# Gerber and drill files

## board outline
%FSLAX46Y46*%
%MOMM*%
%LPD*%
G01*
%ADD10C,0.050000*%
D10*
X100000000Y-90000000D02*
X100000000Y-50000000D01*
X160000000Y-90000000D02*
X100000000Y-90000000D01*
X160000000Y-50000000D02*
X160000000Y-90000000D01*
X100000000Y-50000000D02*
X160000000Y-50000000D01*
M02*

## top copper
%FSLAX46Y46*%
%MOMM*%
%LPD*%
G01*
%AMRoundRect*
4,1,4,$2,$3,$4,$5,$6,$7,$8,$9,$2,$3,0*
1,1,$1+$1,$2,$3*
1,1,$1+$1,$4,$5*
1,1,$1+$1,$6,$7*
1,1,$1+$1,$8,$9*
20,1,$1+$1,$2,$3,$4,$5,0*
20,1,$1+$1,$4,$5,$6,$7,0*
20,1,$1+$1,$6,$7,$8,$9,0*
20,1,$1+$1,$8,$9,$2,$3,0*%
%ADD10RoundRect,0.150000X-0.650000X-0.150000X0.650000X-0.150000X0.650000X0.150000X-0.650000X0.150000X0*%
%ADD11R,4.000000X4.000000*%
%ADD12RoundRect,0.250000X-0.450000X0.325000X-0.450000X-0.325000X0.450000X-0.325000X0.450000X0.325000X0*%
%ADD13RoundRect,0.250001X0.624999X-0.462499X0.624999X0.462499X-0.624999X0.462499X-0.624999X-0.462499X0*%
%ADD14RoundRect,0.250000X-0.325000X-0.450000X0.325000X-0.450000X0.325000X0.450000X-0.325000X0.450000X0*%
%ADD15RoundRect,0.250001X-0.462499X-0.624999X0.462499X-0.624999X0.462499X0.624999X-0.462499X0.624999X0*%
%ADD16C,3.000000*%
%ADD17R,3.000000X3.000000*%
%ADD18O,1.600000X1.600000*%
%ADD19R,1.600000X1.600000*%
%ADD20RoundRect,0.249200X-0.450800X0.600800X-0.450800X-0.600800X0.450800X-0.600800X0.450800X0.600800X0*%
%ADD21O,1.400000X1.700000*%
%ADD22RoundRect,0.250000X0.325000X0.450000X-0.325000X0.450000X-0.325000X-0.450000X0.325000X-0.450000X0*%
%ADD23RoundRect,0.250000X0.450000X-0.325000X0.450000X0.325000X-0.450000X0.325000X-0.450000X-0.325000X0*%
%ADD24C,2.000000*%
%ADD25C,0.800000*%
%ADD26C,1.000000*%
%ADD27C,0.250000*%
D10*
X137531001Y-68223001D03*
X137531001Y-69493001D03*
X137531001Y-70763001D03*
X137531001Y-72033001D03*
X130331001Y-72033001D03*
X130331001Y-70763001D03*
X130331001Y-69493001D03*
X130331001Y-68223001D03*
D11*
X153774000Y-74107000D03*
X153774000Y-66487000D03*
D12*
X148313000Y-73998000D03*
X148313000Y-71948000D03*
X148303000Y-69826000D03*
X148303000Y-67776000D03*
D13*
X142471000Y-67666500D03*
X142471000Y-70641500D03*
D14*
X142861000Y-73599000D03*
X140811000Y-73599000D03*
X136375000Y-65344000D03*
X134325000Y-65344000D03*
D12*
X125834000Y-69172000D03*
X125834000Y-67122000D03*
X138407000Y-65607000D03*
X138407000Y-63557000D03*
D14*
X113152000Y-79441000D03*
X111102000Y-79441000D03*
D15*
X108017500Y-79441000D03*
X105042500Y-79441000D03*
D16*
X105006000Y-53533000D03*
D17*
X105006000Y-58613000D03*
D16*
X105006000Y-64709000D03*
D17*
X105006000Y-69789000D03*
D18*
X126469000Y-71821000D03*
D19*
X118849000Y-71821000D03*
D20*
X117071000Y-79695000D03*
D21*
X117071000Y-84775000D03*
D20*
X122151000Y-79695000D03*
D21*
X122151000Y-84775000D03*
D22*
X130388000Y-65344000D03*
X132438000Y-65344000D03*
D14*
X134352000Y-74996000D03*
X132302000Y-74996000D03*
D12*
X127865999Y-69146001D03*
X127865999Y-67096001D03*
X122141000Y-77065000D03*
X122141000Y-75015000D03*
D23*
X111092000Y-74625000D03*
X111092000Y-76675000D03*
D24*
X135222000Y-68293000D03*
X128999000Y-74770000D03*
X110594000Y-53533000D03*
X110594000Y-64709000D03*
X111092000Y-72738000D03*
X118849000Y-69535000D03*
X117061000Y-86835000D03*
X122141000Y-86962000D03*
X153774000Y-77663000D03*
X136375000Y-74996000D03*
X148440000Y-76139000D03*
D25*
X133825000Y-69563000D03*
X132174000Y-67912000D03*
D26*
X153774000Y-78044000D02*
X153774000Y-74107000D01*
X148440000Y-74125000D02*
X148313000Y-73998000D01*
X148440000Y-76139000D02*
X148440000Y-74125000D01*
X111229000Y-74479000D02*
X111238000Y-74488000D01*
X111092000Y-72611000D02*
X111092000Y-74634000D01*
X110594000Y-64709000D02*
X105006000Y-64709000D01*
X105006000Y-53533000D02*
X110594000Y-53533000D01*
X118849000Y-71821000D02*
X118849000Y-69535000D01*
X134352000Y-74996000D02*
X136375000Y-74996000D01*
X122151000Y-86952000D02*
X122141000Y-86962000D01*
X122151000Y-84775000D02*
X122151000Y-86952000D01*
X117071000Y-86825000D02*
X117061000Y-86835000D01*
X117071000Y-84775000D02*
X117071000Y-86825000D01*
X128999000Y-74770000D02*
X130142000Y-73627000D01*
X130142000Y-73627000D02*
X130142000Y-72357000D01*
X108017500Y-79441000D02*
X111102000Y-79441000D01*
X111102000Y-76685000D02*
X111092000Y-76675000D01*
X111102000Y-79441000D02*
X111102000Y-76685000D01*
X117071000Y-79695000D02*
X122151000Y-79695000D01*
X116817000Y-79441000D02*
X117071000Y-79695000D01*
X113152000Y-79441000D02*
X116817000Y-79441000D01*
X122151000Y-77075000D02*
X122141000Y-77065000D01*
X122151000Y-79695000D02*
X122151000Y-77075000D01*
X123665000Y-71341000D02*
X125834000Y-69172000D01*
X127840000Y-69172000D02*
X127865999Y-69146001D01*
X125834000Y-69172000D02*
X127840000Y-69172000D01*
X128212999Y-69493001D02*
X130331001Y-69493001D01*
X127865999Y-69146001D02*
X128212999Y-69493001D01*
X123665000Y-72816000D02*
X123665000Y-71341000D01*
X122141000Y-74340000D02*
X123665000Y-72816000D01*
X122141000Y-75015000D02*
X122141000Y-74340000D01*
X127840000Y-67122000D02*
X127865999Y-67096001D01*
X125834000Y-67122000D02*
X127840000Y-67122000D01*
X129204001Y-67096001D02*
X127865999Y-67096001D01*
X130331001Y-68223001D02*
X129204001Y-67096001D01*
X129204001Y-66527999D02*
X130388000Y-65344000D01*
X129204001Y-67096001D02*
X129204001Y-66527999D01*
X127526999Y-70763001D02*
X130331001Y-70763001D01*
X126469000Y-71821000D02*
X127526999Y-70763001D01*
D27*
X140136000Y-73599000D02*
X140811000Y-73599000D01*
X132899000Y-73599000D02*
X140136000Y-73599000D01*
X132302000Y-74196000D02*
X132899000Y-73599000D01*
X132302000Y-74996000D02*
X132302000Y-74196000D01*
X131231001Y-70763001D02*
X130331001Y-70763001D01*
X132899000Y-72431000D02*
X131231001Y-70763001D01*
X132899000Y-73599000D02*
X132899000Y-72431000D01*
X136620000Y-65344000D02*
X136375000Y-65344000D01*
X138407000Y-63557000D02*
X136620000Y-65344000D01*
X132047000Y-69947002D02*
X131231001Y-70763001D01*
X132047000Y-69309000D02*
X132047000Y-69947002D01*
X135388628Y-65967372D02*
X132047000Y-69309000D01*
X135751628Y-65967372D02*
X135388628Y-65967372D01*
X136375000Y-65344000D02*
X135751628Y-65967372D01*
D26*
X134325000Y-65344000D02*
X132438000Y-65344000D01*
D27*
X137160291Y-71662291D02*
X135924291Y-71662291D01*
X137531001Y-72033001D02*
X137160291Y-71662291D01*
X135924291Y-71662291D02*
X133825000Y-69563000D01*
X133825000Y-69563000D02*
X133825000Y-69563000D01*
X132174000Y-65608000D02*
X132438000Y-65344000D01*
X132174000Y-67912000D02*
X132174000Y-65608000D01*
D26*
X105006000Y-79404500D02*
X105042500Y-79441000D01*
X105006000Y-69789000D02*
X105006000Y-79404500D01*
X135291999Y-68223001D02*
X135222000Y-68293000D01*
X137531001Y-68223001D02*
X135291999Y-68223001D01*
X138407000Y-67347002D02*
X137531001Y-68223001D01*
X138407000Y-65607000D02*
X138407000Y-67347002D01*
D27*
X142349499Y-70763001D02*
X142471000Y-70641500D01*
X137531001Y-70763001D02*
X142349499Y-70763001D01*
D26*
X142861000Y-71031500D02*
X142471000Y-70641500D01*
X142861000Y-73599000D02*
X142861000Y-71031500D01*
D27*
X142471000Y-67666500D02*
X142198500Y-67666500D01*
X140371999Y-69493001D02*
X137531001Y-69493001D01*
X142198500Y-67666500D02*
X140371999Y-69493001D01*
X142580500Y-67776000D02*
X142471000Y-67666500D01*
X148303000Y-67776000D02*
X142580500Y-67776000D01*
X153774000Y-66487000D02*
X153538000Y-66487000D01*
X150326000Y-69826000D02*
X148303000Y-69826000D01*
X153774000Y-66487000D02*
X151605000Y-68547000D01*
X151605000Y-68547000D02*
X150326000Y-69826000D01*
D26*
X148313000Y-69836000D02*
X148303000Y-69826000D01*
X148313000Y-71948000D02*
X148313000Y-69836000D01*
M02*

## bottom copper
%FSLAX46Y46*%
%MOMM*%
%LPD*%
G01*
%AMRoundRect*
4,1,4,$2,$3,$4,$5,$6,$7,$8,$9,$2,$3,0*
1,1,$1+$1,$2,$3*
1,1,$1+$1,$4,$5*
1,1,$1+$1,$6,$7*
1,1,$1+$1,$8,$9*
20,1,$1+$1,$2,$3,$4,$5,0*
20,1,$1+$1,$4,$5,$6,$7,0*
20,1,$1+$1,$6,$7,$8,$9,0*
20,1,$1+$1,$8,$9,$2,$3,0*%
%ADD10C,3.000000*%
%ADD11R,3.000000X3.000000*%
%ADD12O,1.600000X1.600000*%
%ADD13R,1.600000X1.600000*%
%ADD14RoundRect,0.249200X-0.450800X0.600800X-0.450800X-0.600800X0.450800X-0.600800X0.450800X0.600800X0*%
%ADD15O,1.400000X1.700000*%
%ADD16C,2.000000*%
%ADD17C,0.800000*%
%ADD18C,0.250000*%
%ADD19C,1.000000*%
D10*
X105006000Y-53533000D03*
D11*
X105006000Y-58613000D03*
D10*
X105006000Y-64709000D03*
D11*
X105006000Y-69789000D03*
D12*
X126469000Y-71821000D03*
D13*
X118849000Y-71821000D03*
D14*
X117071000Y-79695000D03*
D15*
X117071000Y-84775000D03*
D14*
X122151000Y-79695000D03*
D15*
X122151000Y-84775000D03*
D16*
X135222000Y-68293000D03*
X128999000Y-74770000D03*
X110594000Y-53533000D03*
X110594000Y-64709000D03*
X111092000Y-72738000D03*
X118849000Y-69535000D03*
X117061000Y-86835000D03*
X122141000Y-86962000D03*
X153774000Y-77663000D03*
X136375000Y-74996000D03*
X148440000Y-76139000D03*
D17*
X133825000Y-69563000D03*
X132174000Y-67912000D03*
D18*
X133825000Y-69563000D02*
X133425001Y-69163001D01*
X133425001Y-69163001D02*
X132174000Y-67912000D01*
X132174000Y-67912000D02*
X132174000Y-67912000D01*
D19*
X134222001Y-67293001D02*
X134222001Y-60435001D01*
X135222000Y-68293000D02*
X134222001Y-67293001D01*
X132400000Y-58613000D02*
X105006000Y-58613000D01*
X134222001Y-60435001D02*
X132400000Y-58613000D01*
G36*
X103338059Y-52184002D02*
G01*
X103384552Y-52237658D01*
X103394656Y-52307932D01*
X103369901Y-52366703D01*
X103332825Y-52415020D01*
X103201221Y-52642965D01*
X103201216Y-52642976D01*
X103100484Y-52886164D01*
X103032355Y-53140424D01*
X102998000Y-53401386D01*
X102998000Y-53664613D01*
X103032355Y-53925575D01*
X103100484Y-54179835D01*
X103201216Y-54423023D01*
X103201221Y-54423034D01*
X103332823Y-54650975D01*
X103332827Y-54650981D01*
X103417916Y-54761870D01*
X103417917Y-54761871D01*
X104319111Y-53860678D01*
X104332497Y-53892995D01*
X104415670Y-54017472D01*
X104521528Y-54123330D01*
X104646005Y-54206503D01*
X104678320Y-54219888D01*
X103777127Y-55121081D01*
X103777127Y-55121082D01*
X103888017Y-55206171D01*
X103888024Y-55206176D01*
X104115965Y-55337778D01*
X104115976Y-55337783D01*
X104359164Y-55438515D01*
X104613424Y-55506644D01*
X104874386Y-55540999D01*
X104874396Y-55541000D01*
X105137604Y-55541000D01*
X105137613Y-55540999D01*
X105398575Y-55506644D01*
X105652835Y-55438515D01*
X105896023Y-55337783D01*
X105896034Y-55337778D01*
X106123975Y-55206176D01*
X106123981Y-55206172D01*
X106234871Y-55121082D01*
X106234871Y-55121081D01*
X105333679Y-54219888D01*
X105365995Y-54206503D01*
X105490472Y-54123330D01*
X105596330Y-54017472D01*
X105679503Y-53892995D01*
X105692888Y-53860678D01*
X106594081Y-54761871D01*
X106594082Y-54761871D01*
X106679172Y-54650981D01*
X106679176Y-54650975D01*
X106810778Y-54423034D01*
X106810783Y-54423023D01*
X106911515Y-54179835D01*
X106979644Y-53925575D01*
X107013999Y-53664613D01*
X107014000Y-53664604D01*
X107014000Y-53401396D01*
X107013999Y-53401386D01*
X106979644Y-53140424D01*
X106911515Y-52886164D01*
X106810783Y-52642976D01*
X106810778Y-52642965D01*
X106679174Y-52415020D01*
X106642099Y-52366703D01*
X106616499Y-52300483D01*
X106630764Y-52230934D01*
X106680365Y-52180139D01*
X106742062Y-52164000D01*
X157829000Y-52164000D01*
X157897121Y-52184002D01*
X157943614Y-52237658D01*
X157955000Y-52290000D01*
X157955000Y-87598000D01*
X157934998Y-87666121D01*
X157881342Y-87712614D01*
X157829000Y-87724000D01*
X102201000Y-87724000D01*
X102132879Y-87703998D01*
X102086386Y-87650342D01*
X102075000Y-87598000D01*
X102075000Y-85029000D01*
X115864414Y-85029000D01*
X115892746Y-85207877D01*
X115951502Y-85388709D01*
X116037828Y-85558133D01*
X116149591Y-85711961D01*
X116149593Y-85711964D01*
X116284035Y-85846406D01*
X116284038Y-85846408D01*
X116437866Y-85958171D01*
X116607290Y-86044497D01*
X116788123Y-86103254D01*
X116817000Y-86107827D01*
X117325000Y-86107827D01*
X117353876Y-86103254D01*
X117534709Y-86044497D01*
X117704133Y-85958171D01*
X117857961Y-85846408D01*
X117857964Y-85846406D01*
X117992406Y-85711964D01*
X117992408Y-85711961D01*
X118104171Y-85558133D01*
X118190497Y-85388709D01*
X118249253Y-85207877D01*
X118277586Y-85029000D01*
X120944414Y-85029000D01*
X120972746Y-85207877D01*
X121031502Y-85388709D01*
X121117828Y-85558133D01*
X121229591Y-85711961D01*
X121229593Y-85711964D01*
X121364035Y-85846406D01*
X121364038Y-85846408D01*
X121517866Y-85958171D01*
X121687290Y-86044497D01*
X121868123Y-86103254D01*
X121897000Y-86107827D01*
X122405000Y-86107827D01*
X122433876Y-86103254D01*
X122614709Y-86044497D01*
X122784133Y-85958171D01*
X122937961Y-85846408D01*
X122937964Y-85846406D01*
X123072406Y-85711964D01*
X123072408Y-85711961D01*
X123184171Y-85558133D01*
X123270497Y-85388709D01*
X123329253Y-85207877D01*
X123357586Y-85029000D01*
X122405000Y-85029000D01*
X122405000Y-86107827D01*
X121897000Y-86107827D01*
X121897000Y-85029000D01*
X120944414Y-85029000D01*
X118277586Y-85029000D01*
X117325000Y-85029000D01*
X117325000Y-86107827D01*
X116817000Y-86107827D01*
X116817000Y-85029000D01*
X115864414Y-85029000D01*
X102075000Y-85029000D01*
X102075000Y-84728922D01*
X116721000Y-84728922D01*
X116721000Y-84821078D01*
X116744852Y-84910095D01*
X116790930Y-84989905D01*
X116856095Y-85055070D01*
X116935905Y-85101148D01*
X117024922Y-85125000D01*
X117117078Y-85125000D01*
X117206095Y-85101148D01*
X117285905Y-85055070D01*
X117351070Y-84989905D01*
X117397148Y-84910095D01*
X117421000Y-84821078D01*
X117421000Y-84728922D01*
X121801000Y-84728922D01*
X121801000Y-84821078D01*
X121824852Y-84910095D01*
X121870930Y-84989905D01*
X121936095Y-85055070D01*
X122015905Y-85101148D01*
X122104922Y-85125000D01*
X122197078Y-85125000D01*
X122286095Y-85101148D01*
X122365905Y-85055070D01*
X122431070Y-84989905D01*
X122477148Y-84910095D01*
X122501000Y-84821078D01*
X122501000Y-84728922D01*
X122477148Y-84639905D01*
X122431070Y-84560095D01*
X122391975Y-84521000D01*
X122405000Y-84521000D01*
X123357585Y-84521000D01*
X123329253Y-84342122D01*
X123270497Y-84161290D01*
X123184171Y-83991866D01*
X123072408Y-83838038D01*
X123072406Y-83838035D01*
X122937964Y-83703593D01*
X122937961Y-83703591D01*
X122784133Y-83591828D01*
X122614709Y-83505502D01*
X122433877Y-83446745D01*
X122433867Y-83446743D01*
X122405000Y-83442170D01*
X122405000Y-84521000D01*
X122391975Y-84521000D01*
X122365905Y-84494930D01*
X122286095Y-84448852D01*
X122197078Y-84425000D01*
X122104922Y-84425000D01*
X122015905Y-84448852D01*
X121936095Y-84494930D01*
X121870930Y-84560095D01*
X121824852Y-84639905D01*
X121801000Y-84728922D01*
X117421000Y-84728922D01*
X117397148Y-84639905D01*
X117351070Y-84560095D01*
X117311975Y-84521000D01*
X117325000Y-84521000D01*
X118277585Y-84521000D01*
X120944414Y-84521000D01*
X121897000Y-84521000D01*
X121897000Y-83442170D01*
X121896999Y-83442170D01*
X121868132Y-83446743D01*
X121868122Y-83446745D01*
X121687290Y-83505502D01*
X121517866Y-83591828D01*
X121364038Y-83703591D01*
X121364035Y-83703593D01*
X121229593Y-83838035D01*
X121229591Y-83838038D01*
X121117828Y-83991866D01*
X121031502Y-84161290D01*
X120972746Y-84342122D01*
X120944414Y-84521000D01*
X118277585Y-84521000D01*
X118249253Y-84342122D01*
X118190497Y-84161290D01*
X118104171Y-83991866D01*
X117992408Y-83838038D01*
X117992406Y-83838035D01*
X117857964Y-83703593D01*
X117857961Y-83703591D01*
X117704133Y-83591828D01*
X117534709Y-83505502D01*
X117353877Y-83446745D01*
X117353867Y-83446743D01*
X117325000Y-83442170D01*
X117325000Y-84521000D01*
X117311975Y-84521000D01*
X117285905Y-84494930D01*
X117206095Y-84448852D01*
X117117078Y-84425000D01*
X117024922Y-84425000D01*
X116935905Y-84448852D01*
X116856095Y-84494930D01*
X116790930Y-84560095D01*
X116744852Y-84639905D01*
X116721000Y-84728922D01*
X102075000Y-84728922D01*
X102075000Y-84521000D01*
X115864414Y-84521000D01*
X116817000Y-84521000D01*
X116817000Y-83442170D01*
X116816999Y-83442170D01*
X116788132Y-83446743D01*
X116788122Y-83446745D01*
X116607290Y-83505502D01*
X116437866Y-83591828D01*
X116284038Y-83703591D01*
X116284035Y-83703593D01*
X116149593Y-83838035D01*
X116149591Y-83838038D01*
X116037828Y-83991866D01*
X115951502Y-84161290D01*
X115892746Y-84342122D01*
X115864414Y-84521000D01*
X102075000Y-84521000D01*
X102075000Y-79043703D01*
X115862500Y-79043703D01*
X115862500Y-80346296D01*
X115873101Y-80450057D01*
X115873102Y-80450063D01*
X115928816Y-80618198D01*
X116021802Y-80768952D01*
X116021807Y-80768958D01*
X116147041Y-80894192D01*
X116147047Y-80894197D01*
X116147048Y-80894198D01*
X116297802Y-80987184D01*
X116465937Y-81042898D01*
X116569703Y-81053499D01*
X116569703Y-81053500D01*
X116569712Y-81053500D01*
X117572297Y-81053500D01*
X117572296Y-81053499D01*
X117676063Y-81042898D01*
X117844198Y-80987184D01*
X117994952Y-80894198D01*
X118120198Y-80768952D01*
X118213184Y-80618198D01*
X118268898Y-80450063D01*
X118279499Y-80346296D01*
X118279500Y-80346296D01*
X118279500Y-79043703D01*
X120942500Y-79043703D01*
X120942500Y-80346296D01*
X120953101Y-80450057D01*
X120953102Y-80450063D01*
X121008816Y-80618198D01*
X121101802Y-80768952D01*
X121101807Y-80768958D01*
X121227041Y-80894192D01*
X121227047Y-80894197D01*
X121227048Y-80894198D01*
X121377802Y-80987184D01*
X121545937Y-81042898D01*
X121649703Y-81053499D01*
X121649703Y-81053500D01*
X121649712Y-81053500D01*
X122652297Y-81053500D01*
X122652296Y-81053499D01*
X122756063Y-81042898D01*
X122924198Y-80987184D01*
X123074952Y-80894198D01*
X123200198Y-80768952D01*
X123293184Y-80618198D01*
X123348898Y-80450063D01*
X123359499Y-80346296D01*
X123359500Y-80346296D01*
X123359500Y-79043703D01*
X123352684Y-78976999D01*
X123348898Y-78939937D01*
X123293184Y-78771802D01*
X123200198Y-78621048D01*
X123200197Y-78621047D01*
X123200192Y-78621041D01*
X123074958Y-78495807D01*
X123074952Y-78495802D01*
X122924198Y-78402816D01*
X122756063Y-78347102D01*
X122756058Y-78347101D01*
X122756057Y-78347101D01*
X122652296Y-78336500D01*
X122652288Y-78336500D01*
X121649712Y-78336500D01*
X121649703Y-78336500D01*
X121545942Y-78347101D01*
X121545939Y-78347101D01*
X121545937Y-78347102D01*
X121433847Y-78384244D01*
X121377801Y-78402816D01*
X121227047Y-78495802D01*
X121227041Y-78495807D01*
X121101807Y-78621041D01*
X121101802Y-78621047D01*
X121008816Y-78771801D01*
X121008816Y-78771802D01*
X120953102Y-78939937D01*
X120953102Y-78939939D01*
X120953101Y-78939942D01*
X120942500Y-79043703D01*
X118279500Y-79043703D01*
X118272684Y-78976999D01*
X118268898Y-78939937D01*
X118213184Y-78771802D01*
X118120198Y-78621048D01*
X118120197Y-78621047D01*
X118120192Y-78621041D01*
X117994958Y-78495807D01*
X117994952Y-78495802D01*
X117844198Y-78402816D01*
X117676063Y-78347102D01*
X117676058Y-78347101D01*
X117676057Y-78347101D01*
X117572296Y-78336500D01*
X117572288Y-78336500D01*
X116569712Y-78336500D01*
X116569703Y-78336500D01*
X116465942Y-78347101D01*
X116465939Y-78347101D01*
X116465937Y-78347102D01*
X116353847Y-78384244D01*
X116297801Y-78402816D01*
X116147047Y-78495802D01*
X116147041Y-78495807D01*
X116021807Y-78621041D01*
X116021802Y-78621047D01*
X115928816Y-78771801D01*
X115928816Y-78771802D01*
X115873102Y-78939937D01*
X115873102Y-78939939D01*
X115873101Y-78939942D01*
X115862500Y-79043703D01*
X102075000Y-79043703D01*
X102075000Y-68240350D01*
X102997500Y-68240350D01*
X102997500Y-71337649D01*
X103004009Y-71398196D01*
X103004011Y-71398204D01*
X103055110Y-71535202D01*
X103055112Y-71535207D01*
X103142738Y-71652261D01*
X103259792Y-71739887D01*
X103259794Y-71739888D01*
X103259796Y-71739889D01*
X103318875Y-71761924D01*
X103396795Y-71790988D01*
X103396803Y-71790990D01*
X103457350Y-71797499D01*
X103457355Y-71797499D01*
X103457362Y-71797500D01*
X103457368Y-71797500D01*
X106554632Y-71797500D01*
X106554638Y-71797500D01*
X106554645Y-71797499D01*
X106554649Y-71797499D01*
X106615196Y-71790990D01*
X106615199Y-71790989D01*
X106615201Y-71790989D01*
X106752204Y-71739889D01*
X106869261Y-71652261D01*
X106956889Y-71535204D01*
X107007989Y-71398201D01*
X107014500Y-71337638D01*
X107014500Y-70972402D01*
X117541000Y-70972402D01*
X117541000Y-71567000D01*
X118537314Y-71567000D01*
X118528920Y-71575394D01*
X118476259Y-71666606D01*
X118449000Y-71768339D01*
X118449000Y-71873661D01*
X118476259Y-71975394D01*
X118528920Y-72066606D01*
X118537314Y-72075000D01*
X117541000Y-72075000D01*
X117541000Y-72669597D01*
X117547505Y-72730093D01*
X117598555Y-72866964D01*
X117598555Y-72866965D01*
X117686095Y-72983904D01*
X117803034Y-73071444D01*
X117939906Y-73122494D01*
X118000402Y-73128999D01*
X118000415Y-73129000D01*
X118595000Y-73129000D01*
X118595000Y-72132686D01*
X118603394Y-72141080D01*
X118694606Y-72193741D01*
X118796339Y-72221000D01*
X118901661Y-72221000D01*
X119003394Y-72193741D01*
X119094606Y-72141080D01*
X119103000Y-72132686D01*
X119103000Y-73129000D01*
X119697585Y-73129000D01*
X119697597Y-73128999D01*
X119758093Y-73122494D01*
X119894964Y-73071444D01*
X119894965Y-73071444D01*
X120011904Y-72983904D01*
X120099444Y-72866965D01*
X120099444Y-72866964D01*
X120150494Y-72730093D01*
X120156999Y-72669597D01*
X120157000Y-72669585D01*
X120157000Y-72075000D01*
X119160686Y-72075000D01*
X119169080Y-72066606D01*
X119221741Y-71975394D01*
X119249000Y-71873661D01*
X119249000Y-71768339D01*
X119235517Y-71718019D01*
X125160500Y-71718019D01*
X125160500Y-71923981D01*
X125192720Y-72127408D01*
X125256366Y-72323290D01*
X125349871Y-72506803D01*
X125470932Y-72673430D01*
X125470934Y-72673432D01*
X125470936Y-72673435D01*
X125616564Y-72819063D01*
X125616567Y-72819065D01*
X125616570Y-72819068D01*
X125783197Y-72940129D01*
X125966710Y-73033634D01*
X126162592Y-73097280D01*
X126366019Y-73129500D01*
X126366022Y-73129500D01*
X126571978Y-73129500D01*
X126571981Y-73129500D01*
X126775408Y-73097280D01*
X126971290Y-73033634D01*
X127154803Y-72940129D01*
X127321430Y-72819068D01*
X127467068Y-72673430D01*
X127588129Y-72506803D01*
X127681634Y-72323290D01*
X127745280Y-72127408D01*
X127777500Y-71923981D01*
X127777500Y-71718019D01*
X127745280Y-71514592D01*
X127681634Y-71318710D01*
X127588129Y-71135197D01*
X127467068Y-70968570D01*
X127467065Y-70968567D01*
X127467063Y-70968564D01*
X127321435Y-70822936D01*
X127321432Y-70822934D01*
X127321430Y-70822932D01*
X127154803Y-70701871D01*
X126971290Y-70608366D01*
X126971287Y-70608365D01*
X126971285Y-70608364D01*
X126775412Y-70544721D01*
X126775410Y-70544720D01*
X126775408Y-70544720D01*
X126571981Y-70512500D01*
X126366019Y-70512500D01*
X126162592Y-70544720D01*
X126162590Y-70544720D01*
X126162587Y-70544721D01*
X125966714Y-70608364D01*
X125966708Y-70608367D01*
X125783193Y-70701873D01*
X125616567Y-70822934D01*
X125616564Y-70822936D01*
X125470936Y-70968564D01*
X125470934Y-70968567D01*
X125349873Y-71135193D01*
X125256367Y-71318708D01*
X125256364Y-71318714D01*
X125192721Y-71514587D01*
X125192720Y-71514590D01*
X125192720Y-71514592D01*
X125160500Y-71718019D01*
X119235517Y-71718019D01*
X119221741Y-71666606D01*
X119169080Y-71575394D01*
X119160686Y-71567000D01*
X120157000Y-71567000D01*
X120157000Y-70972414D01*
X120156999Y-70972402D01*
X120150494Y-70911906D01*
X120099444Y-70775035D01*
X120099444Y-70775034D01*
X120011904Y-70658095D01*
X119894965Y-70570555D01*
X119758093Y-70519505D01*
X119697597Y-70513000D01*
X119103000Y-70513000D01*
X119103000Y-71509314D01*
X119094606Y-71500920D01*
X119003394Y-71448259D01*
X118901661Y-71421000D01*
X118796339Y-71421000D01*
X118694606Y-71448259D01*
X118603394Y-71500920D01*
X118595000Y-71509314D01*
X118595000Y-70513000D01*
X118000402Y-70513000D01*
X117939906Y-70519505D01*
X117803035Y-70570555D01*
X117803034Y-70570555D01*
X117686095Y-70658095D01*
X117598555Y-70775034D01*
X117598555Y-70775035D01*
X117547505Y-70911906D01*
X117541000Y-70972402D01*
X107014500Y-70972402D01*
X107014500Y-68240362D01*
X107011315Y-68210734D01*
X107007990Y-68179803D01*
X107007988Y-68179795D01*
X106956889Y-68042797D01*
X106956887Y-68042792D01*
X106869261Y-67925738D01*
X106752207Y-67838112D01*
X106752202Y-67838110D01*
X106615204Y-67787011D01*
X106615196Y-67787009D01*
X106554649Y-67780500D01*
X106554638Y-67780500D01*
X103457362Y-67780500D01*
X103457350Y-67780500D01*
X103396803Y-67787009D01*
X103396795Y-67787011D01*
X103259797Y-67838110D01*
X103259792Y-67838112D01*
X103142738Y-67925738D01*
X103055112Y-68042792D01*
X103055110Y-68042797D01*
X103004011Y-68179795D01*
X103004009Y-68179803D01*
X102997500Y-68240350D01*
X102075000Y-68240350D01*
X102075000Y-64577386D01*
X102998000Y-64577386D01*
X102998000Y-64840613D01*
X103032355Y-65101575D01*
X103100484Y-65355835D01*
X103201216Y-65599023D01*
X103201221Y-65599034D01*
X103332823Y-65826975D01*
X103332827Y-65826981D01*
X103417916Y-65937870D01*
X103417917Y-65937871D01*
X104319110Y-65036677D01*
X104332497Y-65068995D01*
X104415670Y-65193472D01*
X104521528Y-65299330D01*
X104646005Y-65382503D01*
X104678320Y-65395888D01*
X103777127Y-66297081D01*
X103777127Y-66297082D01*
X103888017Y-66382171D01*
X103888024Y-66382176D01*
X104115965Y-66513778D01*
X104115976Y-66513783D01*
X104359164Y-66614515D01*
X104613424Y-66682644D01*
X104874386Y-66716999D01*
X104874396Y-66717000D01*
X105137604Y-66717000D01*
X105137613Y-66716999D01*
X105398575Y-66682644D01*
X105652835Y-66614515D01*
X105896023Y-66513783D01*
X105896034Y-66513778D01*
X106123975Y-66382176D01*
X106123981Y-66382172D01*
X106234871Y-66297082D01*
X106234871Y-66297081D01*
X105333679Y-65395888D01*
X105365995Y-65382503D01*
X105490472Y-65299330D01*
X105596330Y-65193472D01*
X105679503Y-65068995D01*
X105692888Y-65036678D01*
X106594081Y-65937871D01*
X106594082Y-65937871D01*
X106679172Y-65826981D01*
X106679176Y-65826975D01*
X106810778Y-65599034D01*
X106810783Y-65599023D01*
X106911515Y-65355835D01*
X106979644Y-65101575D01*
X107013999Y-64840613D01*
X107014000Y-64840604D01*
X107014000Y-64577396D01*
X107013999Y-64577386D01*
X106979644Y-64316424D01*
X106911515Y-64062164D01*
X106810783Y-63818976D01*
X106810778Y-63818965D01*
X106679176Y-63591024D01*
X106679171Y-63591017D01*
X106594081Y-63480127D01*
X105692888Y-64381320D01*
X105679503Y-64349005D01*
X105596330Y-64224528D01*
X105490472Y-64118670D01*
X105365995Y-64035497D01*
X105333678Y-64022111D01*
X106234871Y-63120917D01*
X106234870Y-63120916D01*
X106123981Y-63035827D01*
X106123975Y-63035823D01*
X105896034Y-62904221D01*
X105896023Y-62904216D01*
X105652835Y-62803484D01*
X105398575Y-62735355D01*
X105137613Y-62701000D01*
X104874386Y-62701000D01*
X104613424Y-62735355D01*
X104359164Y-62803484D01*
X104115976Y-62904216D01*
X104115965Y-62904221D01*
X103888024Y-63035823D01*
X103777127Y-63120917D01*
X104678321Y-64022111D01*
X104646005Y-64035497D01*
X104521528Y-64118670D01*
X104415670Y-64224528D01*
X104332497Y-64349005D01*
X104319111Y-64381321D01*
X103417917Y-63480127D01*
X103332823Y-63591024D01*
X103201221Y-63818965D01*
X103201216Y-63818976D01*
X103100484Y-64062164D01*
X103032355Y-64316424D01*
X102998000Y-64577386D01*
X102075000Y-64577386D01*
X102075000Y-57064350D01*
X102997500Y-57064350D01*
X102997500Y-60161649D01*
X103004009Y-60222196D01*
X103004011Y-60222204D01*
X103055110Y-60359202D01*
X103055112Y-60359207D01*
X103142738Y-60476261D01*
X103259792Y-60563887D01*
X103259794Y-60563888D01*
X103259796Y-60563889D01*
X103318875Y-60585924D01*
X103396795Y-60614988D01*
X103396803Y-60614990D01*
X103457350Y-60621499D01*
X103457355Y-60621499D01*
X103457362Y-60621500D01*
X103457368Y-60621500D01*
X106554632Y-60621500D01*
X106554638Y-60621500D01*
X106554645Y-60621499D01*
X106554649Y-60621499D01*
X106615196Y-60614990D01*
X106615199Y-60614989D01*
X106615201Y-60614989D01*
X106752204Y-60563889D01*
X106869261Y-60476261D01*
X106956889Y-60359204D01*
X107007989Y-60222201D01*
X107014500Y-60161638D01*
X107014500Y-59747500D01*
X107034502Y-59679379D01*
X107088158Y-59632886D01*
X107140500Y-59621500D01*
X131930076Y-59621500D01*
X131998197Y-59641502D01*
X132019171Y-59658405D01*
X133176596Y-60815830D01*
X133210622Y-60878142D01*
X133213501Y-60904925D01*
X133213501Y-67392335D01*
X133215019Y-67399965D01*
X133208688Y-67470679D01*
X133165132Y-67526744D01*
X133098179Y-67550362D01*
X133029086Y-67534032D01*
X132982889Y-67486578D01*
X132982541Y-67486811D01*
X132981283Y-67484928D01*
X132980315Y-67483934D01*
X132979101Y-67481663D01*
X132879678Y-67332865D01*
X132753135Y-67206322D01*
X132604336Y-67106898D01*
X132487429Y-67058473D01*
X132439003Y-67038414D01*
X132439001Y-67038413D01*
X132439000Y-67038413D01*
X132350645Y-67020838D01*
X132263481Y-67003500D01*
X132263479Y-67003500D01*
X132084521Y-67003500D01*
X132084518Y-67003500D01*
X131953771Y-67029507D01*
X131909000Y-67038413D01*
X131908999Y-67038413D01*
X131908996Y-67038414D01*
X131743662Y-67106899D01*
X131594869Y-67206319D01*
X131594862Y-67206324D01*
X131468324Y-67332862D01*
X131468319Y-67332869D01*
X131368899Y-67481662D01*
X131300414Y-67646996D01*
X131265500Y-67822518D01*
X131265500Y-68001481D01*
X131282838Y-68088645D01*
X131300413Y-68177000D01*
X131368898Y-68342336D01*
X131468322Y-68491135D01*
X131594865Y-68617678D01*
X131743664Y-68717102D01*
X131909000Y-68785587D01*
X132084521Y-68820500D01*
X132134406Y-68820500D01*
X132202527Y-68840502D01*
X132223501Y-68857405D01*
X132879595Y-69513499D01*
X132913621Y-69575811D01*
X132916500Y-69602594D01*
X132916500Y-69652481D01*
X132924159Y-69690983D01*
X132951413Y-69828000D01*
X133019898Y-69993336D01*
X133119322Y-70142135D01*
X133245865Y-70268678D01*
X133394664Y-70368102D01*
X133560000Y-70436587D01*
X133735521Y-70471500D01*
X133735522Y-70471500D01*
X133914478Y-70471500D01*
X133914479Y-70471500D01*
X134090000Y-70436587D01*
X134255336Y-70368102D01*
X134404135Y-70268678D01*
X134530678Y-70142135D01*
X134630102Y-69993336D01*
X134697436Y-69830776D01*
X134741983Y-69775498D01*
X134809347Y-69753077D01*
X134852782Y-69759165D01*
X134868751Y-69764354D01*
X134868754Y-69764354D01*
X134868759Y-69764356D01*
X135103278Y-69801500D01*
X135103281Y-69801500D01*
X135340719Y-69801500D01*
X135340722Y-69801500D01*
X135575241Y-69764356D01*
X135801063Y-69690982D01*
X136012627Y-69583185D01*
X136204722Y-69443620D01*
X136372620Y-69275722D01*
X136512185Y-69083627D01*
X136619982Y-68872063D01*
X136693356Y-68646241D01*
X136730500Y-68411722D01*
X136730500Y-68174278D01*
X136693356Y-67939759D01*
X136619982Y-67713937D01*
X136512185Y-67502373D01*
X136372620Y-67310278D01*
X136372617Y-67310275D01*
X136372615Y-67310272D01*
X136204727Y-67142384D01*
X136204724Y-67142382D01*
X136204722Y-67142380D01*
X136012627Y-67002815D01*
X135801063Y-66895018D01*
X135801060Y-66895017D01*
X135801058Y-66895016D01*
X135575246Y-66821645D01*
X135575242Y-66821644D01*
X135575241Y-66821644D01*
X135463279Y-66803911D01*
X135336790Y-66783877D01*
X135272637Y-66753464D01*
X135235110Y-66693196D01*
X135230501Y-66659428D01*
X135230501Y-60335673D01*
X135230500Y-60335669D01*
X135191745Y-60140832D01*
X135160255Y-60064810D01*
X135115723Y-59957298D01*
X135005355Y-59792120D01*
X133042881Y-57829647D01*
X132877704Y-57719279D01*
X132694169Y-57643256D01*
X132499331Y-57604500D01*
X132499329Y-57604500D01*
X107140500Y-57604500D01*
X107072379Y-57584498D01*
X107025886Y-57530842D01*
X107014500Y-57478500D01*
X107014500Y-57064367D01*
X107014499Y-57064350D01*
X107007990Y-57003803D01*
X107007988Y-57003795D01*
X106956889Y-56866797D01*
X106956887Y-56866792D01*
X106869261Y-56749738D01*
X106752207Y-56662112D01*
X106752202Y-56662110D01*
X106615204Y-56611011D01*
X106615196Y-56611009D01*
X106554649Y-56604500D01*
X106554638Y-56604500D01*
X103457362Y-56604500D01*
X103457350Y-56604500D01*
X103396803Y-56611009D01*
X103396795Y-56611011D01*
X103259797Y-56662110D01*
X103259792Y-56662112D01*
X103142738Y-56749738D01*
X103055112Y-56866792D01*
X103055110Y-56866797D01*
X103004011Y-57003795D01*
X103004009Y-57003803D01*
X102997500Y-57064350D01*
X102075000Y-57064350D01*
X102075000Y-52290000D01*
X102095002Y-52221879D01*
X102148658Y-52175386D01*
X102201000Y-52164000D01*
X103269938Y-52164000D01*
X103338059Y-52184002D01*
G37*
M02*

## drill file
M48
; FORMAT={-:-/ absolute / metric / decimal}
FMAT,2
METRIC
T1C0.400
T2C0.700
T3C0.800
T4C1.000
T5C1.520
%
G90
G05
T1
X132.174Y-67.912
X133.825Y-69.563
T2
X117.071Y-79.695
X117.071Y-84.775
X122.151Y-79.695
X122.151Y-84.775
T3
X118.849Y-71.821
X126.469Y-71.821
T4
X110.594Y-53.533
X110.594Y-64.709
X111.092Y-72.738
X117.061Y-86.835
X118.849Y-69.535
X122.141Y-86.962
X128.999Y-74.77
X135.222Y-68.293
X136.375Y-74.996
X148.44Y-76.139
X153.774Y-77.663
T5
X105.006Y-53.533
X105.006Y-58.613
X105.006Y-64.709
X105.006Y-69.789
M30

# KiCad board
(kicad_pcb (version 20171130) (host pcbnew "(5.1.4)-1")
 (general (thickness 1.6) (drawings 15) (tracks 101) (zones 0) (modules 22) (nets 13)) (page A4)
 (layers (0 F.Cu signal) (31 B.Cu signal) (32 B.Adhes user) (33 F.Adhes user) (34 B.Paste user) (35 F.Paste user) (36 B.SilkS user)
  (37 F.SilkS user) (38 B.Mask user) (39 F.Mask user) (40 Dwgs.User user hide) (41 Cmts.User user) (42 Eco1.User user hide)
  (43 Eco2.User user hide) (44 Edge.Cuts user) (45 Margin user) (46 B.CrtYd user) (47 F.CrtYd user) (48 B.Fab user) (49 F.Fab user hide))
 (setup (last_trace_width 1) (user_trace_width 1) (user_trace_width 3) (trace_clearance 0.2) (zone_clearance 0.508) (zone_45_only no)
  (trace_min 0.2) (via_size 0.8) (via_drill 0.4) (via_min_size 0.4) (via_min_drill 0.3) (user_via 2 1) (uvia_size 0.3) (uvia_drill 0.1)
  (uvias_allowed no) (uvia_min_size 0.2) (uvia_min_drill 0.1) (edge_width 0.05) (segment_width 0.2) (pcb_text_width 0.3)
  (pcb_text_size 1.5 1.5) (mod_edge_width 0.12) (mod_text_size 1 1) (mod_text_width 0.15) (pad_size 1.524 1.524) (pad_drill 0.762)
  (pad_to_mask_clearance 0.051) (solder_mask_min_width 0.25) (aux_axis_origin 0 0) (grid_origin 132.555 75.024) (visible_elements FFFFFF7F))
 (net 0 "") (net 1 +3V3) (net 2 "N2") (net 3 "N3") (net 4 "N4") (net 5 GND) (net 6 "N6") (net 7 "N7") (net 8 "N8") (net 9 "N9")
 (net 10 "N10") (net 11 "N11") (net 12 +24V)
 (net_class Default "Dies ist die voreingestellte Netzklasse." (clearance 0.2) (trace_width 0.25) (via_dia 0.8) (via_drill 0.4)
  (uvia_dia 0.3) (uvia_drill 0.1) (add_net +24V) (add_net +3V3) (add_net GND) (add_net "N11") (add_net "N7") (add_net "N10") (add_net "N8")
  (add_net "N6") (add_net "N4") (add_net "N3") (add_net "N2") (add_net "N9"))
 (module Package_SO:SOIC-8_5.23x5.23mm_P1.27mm (layer F.Cu) (at 133.931001 70.128001)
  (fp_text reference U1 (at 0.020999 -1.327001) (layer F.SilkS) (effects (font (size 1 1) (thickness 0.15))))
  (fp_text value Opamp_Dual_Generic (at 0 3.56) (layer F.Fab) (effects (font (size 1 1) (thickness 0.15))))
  (pad 8 smd roundrect (at 3.6 -1.905) (size 1.6 0.6) (layers F.Cu F.Paste F.Mask) (roundrect_rratio 0.25) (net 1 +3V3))
  (pad 7 smd roundrect (at 3.6 -0.635) (size 1.6 0.6) (layers F.Cu F.Paste F.Mask) (roundrect_rratio 0.25) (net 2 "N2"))
  (pad 6 smd roundrect (at 3.6 0.635) (size 1.6 0.6) (layers F.Cu F.Paste F.Mask) (roundrect_rratio 0.25) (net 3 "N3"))
  (pad 5 smd roundrect (at 3.6 1.905) (size 1.6 0.6) (layers F.Cu F.Paste F.Mask) (roundrect_rratio 0.25) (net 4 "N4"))
  (pad 4 smd roundrect (at -3.6 1.905) (size 1.6 0.6) (layers F.Cu F.Paste F.Mask) (roundrect_rratio 0.25) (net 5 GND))
  (pad 3 smd roundrect (at -3.6 0.635) (size 1.6 0.6) (layers F.Cu F.Paste F.Mask) (roundrect_rratio 0.25) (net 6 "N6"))
  (pad 2 smd roundrect (at -3.6 -0.635) (size 1.6 0.6) (layers F.Cu F.Paste F.Mask) (roundrect_rratio 0.25) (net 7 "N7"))
  (pad 1 smd roundrect (at -3.6 -1.905) (size 1.6 0.6) (layers F.Cu F.Paste F.Mask) (roundrect_rratio 0.25) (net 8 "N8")))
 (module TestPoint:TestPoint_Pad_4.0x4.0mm (layer F.Cu) (at 153.774 74.107)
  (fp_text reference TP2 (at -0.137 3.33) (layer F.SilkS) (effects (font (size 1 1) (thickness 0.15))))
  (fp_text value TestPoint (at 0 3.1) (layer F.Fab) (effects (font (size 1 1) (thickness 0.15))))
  (pad 1 smd rect (at 0 0) (size 4 4) (layers F.Cu F.Mask) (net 5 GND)))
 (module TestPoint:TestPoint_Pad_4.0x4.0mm (layer F.Cu) (at 153.774 66.487)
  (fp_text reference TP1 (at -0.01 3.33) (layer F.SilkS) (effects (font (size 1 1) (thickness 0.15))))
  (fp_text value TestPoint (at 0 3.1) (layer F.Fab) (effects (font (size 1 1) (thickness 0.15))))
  (pad 1 smd rect (at 0 0) (size 4 4) (layers F.Cu F.Mask) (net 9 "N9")))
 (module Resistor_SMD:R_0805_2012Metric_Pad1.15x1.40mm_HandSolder (layer F.Cu) (at 148.313 72.973 270)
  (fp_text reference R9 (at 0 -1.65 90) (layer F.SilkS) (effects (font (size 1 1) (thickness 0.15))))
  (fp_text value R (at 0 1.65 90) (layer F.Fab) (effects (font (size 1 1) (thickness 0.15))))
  (pad 2 smd roundrect (at 1.025 0 270) (size 1.15 1.4) (layers F.Cu F.Paste F.Mask) (roundrect_rratio 0.217391) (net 5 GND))
  (pad 1 smd roundrect (at -1.025 0 270) (size 1.15 1.4) (layers F.Cu F.Paste F.Mask) (roundrect_rratio 0.217391) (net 9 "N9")))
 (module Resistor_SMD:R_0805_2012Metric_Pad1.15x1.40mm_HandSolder (layer F.Cu) (at 148.303 68.801 270)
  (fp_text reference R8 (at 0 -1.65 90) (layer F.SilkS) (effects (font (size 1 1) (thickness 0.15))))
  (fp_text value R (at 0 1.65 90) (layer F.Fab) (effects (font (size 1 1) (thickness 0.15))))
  (pad 2 smd roundrect (at 1.025 0 270) (size 1.15 1.4) (layers F.Cu F.Paste F.Mask) (roundrect_rratio 0.217391) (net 9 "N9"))
  (pad 1 smd roundrect (at -1.025 0 270) (size 1.15 1.4) (layers F.Cu F.Paste F.Mask) (roundrect_rratio 0.217391) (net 2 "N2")))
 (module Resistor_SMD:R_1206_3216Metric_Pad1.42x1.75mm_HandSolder (layer F.Cu) (at 142.471 69.154 90)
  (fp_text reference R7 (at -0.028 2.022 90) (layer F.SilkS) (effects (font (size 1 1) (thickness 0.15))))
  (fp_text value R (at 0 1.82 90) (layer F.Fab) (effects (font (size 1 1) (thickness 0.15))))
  (pad 2 smd roundrect (at 1.4875 0 90) (size 1.425 1.75) (layers F.Cu F.Paste F.Mask) (roundrect_rratio 0.175439) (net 2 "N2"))
  (pad 1 smd roundrect (at -1.4875 0 90) (size 1.425 1.75) (layers F.Cu F.Paste F.Mask) (roundrect_rratio 0.175439) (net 3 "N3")))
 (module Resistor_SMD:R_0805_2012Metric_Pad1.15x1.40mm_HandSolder (layer F.Cu) (at 141.836 73.599)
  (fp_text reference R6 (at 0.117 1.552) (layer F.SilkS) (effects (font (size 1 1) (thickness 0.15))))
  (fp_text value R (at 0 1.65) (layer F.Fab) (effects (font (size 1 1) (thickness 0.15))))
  (pad 2 smd roundrect (at 1.025 0) (size 1.15 1.4) (layers F.Cu F.Paste F.Mask) (roundrect_rratio 0.217391) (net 3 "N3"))
  (pad 1 smd roundrect (at -1.025 0) (size 1.15 1.4) (layers F.Cu F.Paste F.Mask) (roundrect_rratio 0.217391) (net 6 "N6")))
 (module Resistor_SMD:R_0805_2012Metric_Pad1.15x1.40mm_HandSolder (layer F.Cu) (at 135.35 65.344)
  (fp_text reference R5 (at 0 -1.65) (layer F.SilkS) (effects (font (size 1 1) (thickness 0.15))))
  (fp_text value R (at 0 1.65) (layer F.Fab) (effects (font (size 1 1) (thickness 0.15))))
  (pad 2 smd roundrect (at 1.025 0) (size 1.15 1.4) (layers F.Cu F.Paste F.Mask) (roundrect_rratio 0.217391) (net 6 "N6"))
  (pad 1 smd roundrect (at -1.025 0) (size 1.15 1.4) (layers F.Cu F.Paste F.Mask) (roundrect_rratio 0.217391) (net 4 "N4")))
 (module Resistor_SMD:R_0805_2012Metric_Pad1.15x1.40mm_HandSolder (layer F.Cu) (at 125.834 68.147 270)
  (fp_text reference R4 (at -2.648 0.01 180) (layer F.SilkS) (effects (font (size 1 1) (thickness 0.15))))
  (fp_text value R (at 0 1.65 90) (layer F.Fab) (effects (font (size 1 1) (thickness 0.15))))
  (pad 2 smd roundrect (at 1.025 0 270) (size 1.15 1.4) (layers F.Cu F.Paste F.Mask) (roundrect_rratio 0.217391) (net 7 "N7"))
  (pad 1 smd roundrect (at -1.025 0 270) (size 1.15 1.4) (layers F.Cu F.Paste F.Mask) (roundrect_rratio 0.217391) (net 8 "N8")))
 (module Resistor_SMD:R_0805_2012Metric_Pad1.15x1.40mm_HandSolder (layer F.Cu) (at 138.407 64.582 270)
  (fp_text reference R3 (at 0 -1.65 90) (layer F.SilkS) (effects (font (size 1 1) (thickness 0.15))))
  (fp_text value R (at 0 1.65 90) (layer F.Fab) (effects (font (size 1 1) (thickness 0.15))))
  (pad 2 smd roundrect (at 1.025 0 270) (size 1.15 1.4) (layers F.Cu F.Paste F.Mask) (roundrect_rratio 0.217391) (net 1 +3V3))
  (pad 1 smd roundrect (at -1.025 0 270) (size 1.15 1.4) (layers F.Cu F.Paste F.Mask) (roundrect_rratio 0.217391) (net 6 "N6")))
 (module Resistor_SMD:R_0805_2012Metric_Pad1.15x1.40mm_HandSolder (layer F.Cu) (at 112.127 79.441)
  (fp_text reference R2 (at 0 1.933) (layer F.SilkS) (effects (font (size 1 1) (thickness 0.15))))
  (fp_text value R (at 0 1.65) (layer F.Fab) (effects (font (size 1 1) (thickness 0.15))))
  (pad 2 smd roundrect (at 1.025 0) (size 1.15 1.4) (layers F.Cu F.Paste F.Mask) (roundrect_rratio 0.217391) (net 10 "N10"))
  (pad 1 smd roundrect (at -1.025 0) (size 1.15 1.4) (layers F.Cu F.Paste F.Mask) (roundrect_rratio 0.217391) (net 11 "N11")))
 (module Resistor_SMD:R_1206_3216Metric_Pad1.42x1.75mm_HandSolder (layer F.Cu) (at 106.53 79.441)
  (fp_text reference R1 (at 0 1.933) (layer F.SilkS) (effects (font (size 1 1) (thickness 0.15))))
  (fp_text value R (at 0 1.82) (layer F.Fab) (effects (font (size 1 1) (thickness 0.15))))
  (pad 2 smd roundrect (at 1.4875 0) (size 1.425 1.75) (layers F.Cu F.Paste F.Mask) (roundrect_rratio 0.175439) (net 11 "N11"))
  (pad 1 smd roundrect (at -1.4875 0) (size 1.425 1.75) (layers F.Cu F.Paste F.Mask) (roundrect_rratio 0.175439) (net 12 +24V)))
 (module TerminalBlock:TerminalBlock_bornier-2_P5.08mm (layer F.Cu) (at 105.006 58.613 90)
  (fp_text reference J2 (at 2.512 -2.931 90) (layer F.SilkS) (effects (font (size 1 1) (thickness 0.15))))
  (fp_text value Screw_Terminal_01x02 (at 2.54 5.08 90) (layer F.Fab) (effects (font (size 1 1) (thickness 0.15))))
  (pad 2 thru_hole circle (at 5.08 0 90) (size 3 3) (drill 1.52) (layers *.Cu *.Mask) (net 5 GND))
  (pad 1 thru_hole rect (at 0 0 90) (size 3 3) (drill 1.52) (layers *.Cu *.Mask) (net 1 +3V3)))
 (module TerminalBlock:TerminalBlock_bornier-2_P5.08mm (layer F.Cu) (at 105.006 69.789 90)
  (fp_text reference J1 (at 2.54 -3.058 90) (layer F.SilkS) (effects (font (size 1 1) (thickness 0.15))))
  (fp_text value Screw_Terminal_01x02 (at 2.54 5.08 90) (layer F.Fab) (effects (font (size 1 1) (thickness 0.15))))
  (pad 2 thru_hole circle (at 5.08 0 90) (size 3 3) (drill 1.52) (layers *.Cu *.Mask) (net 5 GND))
  (pad 1 thru_hole rect (at 0 0 90) (size 3 3) (drill 1.52) (layers *.Cu *.Mask) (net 12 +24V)))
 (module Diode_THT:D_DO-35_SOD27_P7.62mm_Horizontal (layer F.Cu) (at 118.849 71.821)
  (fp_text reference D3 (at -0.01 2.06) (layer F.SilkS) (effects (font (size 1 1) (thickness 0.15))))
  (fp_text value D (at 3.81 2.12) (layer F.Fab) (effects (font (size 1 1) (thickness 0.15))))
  (pad 2 thru_hole oval (at 7.62 0) (size 1.6 1.6) (drill 0.8) (layers *.Cu *.Mask) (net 6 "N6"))
  (pad 1 thru_hole rect (at 0 0) (size 1.6 1.6) (drill 0.8) (layers *.Cu *.Mask) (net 5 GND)))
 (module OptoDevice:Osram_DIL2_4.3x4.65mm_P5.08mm (layer F.Cu) (at 117.071 79.695 270)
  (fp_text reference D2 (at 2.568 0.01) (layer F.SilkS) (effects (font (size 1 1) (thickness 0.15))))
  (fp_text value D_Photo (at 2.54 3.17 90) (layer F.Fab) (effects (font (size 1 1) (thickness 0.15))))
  (pad 1 thru_hole roundrect (at 0 0 270) (size 1.7 1.4) (drill 0.7) (layers *.Cu *.Mask) (roundrect_rratio 0.178) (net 10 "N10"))
  (pad 2 thru_hole oval (at 5.08 0 270) (size 1.7 1.4) (drill 0.7) (layers *.Cu *.Mask) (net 5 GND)))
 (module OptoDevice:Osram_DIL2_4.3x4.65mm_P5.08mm (layer F.Cu) (at 122.151 79.695 270)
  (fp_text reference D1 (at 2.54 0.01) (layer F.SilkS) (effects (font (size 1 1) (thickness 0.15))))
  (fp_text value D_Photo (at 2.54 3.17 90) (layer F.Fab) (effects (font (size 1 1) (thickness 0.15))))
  (pad 1 thru_hole roundrect (at 0 0 270) (size 1.7 1.4) (drill 0.7) (layers *.Cu *.Mask) (roundrect_rratio 0.178) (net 10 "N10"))
  (pad 2 thru_hole oval (at 5.08 0 270) (size 1.7 1.4) (drill 0.7) (layers *.Cu *.Mask) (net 5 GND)))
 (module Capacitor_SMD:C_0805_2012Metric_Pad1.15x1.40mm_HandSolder (layer F.Cu) (at 131.413 65.344 180)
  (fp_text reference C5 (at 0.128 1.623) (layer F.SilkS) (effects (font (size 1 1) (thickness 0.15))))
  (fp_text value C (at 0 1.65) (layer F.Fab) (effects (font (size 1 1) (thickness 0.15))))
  (pad 2 smd roundrect (at 1.025 0 180) (size 1.15 1.4) (layers F.Cu F.Paste F.Mask) (roundrect_rratio 0.217391) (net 8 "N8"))
  (pad 1 smd roundrect (at -1.025 0 180) (size 1.15 1.4) (layers F.Cu F.Paste F.Mask) (roundrect_rratio 0.217391) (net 4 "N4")))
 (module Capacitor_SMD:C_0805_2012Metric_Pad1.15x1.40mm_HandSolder (layer F.Cu) (at 133.327 74.996)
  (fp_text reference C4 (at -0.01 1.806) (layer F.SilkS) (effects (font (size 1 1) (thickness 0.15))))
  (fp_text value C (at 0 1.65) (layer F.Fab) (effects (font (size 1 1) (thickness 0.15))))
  (pad 2 smd roundrect (at 1.025 0) (size 1.15 1.4) (layers F.Cu F.Paste F.Mask) (roundrect_rratio 0.217391) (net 5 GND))
  (pad 1 smd roundrect (at -1.025 0) (size 1.15 1.4) (layers F.Cu F.Paste F.Mask) (roundrect_rratio 0.217391) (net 6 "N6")))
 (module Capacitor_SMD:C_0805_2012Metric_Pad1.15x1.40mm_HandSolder (layer F.Cu) (at 127.865999 68.121001 270)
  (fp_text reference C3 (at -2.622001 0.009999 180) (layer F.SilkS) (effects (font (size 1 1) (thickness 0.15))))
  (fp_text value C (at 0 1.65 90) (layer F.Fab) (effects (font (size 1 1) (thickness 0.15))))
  (pad 2 smd roundrect (at 1.025 0 270) (size 1.15 1.4) (layers F.Cu F.Paste F.Mask) (roundrect_rratio 0.217391) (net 7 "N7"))
  (pad 1 smd roundrect (at -1.025 0 270) (size 1.15 1.4) (layers F.Cu F.Paste F.Mask) (roundrect_rratio 0.217391) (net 8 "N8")))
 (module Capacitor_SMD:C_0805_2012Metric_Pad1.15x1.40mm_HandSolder (layer F.Cu) (at 122.141 76.04 270)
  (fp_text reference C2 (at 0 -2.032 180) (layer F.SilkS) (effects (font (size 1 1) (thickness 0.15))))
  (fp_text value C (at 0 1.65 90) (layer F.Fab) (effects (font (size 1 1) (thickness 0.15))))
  (pad 2 smd roundrect (at 1.025 0 270) (size 1.15 1.4) (layers F.Cu F.Paste F.Mask) (roundrect_rratio 0.217391) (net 10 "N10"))
  (pad 1 smd roundrect (at -1.025 0 270) (size 1.15 1.4) (layers F.Cu F.Paste F.Mask) (roundrect_rratio 0.217391) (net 7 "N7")))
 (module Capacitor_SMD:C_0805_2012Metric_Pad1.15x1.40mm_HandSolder (layer F.Cu) (at 111.092 75.65 90)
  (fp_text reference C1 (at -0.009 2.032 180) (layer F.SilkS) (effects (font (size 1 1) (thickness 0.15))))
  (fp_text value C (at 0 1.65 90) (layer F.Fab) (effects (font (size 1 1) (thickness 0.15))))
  (pad 2 smd roundrect (at 1.025 0 90) (size 1.15 1.4) (layers F.Cu F.Paste F.Mask) (roundrect_rratio 0.217391) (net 5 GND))
  (pad 1 smd roundrect (at -1.025 0 90) (size 1.15 1.4) (layers F.Cu F.Paste F.Mask) (roundrect_rratio 0.217391) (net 11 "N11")))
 (gr_line (start 100 90) (end 100 50) (layer Edge.Cuts) (width 0.05))
 (gr_line (start 160 90) (end 100 90) (layer Edge.Cuts) (width 0.05))
 (gr_line (start 160 50) (end 160 90) (layer Edge.Cuts) (width 0.05))
 (gr_line (start 100 50) (end 160 50) (layer Edge.Cuts) (width 0.05))
 (via (at 135.222 68.293) (size 2) (drill 1) (layers F.Cu B.Cu) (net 1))
 (via (at 128.999 74.77) (size 2) (drill 1) (layers F.Cu B.Cu) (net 5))
 (via (at 110.594 53.533) (size 2) (drill 1) (layers F.Cu B.Cu) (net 5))
 (via (at 110.594 64.709) (size 2) (drill 1) (layers F.Cu B.Cu) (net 5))
 (via (at 111.092 72.738) (size 2) (drill 1) (layers F.Cu B.Cu) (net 5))
 (via (at 118.849 69.535) (size 2) (drill 1) (layers F.Cu B.Cu) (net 5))
 (via (at 117.061 86.835) (size 2) (drill 1) (layers F.Cu B.Cu) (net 5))
 (via (at 122.141 86.962) (size 2) (drill 1) (layers F.Cu B.Cu) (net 5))
 (via (at 153.774 77.663) (size 2) (drill 1) (layers F.Cu B.Cu) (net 5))
 (via (at 136.375 74.996) (size 2) (drill 1) (layers F.Cu B.Cu) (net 5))
 (via (at 148.44 76.139) (size 2) (drill 1) (layers F.Cu B.Cu) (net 5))
 (segment (start 153.774 78.044) (end 153.774 74.107) (width 1) (layer F.Cu) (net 5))
 (segment (start 148.44 74.125) (end 148.313 73.998) (width 1) (layer F.Cu) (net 5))
 (segment (start 148.44 76.139) (end 148.44 74.125) (width 1) (layer F.Cu) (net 5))
 (segment (start 111.229 74.479) (end 111.238 74.488) (width 1) (layer F.Cu) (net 5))
 (segment (start 111.092 72.611) (end 111.092 74.634) (width 1) (layer F.Cu) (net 5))
 (segment (start 110.594 64.709) (end 105.006 64.709) (width 1) (layer F.Cu) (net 5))
 (segment (start 105.006 53.533) (end 110.594 53.533) (width 1) (layer F.Cu) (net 5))
 (segment (start 118.849 71.821) (end 118.849 69.535) (width 1) (layer F.Cu) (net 5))
 (segment (start 134.352 74.996) (end 136.375 74.996) (width 1) (layer F.Cu) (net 5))
 (segment (start 122.151 86.952) (end 122.141 86.962) (width 1) (layer F.Cu) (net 5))
 (segment (start 122.151 84.775) (end 122.151 86.952) (width 1) (layer F.Cu) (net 5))
 (segment (start 117.071 86.825) (end 117.061 86.835) (width 1) (layer F.Cu) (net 5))
 (segment (start 117.071 84.775) (end 117.071 86.825) (width 1) (layer F.Cu) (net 5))
 (segment (start 128.999 74.77) (end 130.142 73.627) (width 1) (layer F.Cu) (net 5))
 (segment (start 130.142 73.627) (end 130.142 72.357) (width 1) (layer F.Cu) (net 5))
 (segment (start 108.0175 79.441) (end 111.102 79.441) (width 1) (layer F.Cu) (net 11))
 (segment (start 111.102 76.685) (end 111.092 76.675) (width 1) (layer F.Cu) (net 11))
 (segment (start 111.102 79.441) (end 111.102 76.685) (width 1) (layer F.Cu) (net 11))
 (segment (start 117.071 79.695) (end 122.151 79.695) (width 1) (layer F.Cu) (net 10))
 (segment (start 116.817 79.441) (end 117.071 79.695) (width 1) (layer F.Cu) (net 10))
 (segment (start 113.152 79.441) (end 116.817 79.441) (width 1) (layer F.Cu) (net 10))
 (segment (start 122.151 77.075) (end 122.141 77.065) (width 1) (layer F.Cu) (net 10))
 (segment (start 122.151 79.695) (end 122.151 77.075) (width 1) (layer F.Cu) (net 10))
 (segment (start 123.665 71.341) (end 125.834 69.172) (width 1) (layer F.Cu) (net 7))
 (segment (start 127.84 69.172) (end 127.865999 69.146001) (width 1) (layer F.Cu) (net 7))
 (segment (start 125.834 69.172) (end 127.84 69.172) (width 1) (layer F.Cu) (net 7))
 (segment (start 128.212999 69.493001) (end 130.331001 69.493001) (width 1) (layer F.Cu) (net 7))
 (segment (start 127.865999 69.146001) (end 128.212999 69.493001) (width 1) (layer F.Cu) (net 7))
 (segment (start 123.665 72.816) (end 123.665 71.341) (width 1) (layer F.Cu) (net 7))
 (segment (start 122.141 74.34) (end 123.665 72.816) (width 1) (layer F.Cu) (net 7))
 (segment (start 122.141 75.015) (end 122.141 74.34) (width 1) (layer F.Cu) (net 7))
 (segment (start 127.84 67.122) (end 127.865999 67.096001) (width 1) (layer F.Cu) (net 8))
 (segment (start 125.834 67.122) (end 127.84 67.122) (width 1) (layer F.Cu) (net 8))
 (segment (start 129.204001 67.096001) (end 127.865999 67.096001) (width 1) (layer F.Cu) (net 8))
 (segment (start 130.331001 68.223001) (end 129.204001 67.096001) (width 1) (layer F.Cu) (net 8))
 (segment (start 129.204001 66.527999) (end 130.388 65.344) (width 1) (layer F.Cu) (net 8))
 (segment (start 129.204001 67.096001) (end 129.204001 66.527999) (width 1) (layer F.Cu) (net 8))
 (segment (start 127.526999 70.763001) (end 130.331001 70.763001) (width 1) (layer F.Cu) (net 6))
 (segment (start 126.469 71.821) (end 127.526999 70.763001) (width 1) (layer F.Cu) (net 6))
 (segment (start 140.136 73.599) (end 140.811 73.599) (width 0.25) (layer F.Cu) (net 6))
 (segment (start 132.899 73.599) (end 140.136 73.599) (width 0.25) (layer F.Cu) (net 6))
 (segment (start 132.302 74.196) (end 132.899 73.599) (width 0.25) (layer F.Cu) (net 6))
 (segment (start 132.302 74.996) (end 132.302 74.196) (width 0.25) (layer F.Cu) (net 6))
 (segment (start 131.231001 70.763001) (end 130.331001 70.763001) (width 0.25) (layer F.Cu) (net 6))
 (segment (start 132.899 72.431) (end 131.231001 70.763001) (width 0.25) (layer F.Cu) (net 6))
 (segment (start 132.899 73.599) (end 132.899 72.431) (width 0.25) (layer F.Cu) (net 6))
 (segment (start 136.62 65.344) (end 136.375 65.344) (width 0.25) (layer F.Cu) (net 6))
 (segment (start 138.407 63.557) (end 136.62 65.344) (width 0.25) (layer F.Cu) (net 6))
 (segment (start 132.047 69.947002) (end 131.231001 70.763001) (width 0.25) (layer F.Cu) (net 6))
 (segment (start 132.047 69.309) (end 132.047 69.947002) (width 0.25) (layer F.Cu) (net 6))
 (segment (start 135.388628 65.967372) (end 132.047 69.309) (width 0.25) (layer F.Cu) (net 6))
 (segment (start 135.751628 65.967372) (end 135.388628 65.967372) (width 0.25) (layer F.Cu) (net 6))
 (segment (start 136.375 65.344) (end 135.751628 65.967372) (width 0.25) (layer F.Cu) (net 6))
 (segment (start 134.325 65.344) (end 132.438 65.344) (width 1) (layer F.Cu) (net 4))
 (segment (start 137.160291 71.662291) (end 135.924291 71.662291) (width 0.25) (layer F.Cu) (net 4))
 (segment (start 137.531001 72.033001) (end 137.160291 71.662291) (width 0.25) (layer F.Cu) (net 4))
 (segment (start 135.924291 71.662291) (end 133.825 69.563) (width 0.25) (layer F.Cu) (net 4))
 (segment (start 133.825 69.563) (end 133.825 69.563) (width 0.25) (layer F.Cu) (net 4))
 (via (at 133.825 69.563) (size 0.8) (drill 0.4) (layers F.Cu B.Cu) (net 4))
 (segment (start 133.825 69.563) (end 133.425001 69.163001) (width 0.25) (layer B.Cu) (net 4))
 (segment (start 133.425001 69.163001) (end 132.174 67.912) (width 0.25) (layer B.Cu) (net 4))
 (segment (start 132.174 67.912) (end 132.174 67.912) (width 0.25) (layer B.Cu) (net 4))
 (via (at 132.174 67.912) (size 0.8) (drill 0.4) (layers F.Cu B.Cu) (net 4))
 (segment (start 132.174 65.608) (end 132.438 65.344) (width 0.25) (layer F.Cu) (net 4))
 (segment (start 132.174 67.912) (end 132.174 65.608) (width 0.25) (layer F.Cu) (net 4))
 (segment (start 105.006 79.4045) (end 105.0425 79.441) (width 1) (layer F.Cu) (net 12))
 (segment (start 105.006 69.789) (end 105.006 79.4045) (width 1) (layer F.Cu) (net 12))
 (segment (start 135.291999 68.223001) (end 135.222 68.293) (width 1) (layer F.Cu) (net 1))
 (segment (start 137.531001 68.223001) (end 135.291999 68.223001) (width 1) (layer F.Cu) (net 1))
 (segment (start 134.222001 67.293001) (end 134.222001 60.435001) (width 1) (layer B.Cu) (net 1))
 (segment (start 135.222 68.293) (end 134.222001 67.293001) (width 1) (layer B.Cu) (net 1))
 (segment (start 132.4 58.613) (end 105.006 58.613) (width 1) (layer B.Cu) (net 1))
 (segment (start 134.222001 60.435001) (end 132.4 58.613) (width 1) (layer B.Cu) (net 1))
 (segment (start 138.407 67.347002) (end 137.531001 68.223001) (width 1) (layer F.Cu) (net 1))
 (segment (start 138.407 65.607) (end 138.407 67.347002) (width 1) (layer F.Cu) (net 1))
 (segment (start 142.349499 70.763001) (end 142.471 70.6415) (width 0.25) (layer F.Cu) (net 3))
 (segment (start 137.531001 70.763001) (end 142.349499 70.763001) (width 0.25) (layer F.Cu) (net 3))
 (segment (start 142.861 71.0315) (end 142.471 70.6415) (width 1) (layer F.Cu) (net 3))
 (segment (start 142.861 73.599) (end 142.861 71.0315) (width 1) (layer F.Cu) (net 3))
 (segment (start 142.471 67.6665) (end 142.1985 67.6665) (width 0.25) (layer F.Cu) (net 2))
 (segment (start 140.371999 69.493001) (end 137.531001 69.493001) (width 0.25) (layer F.Cu) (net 2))
 (segment (start 142.1985 67.6665) (end 140.371999 69.493001) (width 0.25) (layer F.Cu) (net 2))
 (segment (start 142.5805 67.776) (end 142.471 67.6665) (width 0.25) (layer F.Cu) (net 2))
 (segment (start 148.303 67.776) (end 142.5805 67.776) (width 0.25) (layer F.Cu) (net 2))
 (segment (start 153.774 66.487) (end 153.538 66.487) (width 0.25) (layer F.Cu) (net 9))
 (segment (start 150.326 69.826) (end 148.303 69.826) (width 0.25) (layer F.Cu) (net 9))
 (segment (start 153.774 66.487) (end 151.605 68.547) (width 0.25) (layer F.Cu) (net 9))
 (segment (start 151.605 68.547) (end 150.326 69.826) (width 0.25) (layer F.Cu) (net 9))
 (segment (start 148.313 69.836) (end 148.303 69.826) (width 1) (layer F.Cu) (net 9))
 (segment (start 148.313 71.948) (end 148.313 69.836) (width 1) (layer F.Cu) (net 9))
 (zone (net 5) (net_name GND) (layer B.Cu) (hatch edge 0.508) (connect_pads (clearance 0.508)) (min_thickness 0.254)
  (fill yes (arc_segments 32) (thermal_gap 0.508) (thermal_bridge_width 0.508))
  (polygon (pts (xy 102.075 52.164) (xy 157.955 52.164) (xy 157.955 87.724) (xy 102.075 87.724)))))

